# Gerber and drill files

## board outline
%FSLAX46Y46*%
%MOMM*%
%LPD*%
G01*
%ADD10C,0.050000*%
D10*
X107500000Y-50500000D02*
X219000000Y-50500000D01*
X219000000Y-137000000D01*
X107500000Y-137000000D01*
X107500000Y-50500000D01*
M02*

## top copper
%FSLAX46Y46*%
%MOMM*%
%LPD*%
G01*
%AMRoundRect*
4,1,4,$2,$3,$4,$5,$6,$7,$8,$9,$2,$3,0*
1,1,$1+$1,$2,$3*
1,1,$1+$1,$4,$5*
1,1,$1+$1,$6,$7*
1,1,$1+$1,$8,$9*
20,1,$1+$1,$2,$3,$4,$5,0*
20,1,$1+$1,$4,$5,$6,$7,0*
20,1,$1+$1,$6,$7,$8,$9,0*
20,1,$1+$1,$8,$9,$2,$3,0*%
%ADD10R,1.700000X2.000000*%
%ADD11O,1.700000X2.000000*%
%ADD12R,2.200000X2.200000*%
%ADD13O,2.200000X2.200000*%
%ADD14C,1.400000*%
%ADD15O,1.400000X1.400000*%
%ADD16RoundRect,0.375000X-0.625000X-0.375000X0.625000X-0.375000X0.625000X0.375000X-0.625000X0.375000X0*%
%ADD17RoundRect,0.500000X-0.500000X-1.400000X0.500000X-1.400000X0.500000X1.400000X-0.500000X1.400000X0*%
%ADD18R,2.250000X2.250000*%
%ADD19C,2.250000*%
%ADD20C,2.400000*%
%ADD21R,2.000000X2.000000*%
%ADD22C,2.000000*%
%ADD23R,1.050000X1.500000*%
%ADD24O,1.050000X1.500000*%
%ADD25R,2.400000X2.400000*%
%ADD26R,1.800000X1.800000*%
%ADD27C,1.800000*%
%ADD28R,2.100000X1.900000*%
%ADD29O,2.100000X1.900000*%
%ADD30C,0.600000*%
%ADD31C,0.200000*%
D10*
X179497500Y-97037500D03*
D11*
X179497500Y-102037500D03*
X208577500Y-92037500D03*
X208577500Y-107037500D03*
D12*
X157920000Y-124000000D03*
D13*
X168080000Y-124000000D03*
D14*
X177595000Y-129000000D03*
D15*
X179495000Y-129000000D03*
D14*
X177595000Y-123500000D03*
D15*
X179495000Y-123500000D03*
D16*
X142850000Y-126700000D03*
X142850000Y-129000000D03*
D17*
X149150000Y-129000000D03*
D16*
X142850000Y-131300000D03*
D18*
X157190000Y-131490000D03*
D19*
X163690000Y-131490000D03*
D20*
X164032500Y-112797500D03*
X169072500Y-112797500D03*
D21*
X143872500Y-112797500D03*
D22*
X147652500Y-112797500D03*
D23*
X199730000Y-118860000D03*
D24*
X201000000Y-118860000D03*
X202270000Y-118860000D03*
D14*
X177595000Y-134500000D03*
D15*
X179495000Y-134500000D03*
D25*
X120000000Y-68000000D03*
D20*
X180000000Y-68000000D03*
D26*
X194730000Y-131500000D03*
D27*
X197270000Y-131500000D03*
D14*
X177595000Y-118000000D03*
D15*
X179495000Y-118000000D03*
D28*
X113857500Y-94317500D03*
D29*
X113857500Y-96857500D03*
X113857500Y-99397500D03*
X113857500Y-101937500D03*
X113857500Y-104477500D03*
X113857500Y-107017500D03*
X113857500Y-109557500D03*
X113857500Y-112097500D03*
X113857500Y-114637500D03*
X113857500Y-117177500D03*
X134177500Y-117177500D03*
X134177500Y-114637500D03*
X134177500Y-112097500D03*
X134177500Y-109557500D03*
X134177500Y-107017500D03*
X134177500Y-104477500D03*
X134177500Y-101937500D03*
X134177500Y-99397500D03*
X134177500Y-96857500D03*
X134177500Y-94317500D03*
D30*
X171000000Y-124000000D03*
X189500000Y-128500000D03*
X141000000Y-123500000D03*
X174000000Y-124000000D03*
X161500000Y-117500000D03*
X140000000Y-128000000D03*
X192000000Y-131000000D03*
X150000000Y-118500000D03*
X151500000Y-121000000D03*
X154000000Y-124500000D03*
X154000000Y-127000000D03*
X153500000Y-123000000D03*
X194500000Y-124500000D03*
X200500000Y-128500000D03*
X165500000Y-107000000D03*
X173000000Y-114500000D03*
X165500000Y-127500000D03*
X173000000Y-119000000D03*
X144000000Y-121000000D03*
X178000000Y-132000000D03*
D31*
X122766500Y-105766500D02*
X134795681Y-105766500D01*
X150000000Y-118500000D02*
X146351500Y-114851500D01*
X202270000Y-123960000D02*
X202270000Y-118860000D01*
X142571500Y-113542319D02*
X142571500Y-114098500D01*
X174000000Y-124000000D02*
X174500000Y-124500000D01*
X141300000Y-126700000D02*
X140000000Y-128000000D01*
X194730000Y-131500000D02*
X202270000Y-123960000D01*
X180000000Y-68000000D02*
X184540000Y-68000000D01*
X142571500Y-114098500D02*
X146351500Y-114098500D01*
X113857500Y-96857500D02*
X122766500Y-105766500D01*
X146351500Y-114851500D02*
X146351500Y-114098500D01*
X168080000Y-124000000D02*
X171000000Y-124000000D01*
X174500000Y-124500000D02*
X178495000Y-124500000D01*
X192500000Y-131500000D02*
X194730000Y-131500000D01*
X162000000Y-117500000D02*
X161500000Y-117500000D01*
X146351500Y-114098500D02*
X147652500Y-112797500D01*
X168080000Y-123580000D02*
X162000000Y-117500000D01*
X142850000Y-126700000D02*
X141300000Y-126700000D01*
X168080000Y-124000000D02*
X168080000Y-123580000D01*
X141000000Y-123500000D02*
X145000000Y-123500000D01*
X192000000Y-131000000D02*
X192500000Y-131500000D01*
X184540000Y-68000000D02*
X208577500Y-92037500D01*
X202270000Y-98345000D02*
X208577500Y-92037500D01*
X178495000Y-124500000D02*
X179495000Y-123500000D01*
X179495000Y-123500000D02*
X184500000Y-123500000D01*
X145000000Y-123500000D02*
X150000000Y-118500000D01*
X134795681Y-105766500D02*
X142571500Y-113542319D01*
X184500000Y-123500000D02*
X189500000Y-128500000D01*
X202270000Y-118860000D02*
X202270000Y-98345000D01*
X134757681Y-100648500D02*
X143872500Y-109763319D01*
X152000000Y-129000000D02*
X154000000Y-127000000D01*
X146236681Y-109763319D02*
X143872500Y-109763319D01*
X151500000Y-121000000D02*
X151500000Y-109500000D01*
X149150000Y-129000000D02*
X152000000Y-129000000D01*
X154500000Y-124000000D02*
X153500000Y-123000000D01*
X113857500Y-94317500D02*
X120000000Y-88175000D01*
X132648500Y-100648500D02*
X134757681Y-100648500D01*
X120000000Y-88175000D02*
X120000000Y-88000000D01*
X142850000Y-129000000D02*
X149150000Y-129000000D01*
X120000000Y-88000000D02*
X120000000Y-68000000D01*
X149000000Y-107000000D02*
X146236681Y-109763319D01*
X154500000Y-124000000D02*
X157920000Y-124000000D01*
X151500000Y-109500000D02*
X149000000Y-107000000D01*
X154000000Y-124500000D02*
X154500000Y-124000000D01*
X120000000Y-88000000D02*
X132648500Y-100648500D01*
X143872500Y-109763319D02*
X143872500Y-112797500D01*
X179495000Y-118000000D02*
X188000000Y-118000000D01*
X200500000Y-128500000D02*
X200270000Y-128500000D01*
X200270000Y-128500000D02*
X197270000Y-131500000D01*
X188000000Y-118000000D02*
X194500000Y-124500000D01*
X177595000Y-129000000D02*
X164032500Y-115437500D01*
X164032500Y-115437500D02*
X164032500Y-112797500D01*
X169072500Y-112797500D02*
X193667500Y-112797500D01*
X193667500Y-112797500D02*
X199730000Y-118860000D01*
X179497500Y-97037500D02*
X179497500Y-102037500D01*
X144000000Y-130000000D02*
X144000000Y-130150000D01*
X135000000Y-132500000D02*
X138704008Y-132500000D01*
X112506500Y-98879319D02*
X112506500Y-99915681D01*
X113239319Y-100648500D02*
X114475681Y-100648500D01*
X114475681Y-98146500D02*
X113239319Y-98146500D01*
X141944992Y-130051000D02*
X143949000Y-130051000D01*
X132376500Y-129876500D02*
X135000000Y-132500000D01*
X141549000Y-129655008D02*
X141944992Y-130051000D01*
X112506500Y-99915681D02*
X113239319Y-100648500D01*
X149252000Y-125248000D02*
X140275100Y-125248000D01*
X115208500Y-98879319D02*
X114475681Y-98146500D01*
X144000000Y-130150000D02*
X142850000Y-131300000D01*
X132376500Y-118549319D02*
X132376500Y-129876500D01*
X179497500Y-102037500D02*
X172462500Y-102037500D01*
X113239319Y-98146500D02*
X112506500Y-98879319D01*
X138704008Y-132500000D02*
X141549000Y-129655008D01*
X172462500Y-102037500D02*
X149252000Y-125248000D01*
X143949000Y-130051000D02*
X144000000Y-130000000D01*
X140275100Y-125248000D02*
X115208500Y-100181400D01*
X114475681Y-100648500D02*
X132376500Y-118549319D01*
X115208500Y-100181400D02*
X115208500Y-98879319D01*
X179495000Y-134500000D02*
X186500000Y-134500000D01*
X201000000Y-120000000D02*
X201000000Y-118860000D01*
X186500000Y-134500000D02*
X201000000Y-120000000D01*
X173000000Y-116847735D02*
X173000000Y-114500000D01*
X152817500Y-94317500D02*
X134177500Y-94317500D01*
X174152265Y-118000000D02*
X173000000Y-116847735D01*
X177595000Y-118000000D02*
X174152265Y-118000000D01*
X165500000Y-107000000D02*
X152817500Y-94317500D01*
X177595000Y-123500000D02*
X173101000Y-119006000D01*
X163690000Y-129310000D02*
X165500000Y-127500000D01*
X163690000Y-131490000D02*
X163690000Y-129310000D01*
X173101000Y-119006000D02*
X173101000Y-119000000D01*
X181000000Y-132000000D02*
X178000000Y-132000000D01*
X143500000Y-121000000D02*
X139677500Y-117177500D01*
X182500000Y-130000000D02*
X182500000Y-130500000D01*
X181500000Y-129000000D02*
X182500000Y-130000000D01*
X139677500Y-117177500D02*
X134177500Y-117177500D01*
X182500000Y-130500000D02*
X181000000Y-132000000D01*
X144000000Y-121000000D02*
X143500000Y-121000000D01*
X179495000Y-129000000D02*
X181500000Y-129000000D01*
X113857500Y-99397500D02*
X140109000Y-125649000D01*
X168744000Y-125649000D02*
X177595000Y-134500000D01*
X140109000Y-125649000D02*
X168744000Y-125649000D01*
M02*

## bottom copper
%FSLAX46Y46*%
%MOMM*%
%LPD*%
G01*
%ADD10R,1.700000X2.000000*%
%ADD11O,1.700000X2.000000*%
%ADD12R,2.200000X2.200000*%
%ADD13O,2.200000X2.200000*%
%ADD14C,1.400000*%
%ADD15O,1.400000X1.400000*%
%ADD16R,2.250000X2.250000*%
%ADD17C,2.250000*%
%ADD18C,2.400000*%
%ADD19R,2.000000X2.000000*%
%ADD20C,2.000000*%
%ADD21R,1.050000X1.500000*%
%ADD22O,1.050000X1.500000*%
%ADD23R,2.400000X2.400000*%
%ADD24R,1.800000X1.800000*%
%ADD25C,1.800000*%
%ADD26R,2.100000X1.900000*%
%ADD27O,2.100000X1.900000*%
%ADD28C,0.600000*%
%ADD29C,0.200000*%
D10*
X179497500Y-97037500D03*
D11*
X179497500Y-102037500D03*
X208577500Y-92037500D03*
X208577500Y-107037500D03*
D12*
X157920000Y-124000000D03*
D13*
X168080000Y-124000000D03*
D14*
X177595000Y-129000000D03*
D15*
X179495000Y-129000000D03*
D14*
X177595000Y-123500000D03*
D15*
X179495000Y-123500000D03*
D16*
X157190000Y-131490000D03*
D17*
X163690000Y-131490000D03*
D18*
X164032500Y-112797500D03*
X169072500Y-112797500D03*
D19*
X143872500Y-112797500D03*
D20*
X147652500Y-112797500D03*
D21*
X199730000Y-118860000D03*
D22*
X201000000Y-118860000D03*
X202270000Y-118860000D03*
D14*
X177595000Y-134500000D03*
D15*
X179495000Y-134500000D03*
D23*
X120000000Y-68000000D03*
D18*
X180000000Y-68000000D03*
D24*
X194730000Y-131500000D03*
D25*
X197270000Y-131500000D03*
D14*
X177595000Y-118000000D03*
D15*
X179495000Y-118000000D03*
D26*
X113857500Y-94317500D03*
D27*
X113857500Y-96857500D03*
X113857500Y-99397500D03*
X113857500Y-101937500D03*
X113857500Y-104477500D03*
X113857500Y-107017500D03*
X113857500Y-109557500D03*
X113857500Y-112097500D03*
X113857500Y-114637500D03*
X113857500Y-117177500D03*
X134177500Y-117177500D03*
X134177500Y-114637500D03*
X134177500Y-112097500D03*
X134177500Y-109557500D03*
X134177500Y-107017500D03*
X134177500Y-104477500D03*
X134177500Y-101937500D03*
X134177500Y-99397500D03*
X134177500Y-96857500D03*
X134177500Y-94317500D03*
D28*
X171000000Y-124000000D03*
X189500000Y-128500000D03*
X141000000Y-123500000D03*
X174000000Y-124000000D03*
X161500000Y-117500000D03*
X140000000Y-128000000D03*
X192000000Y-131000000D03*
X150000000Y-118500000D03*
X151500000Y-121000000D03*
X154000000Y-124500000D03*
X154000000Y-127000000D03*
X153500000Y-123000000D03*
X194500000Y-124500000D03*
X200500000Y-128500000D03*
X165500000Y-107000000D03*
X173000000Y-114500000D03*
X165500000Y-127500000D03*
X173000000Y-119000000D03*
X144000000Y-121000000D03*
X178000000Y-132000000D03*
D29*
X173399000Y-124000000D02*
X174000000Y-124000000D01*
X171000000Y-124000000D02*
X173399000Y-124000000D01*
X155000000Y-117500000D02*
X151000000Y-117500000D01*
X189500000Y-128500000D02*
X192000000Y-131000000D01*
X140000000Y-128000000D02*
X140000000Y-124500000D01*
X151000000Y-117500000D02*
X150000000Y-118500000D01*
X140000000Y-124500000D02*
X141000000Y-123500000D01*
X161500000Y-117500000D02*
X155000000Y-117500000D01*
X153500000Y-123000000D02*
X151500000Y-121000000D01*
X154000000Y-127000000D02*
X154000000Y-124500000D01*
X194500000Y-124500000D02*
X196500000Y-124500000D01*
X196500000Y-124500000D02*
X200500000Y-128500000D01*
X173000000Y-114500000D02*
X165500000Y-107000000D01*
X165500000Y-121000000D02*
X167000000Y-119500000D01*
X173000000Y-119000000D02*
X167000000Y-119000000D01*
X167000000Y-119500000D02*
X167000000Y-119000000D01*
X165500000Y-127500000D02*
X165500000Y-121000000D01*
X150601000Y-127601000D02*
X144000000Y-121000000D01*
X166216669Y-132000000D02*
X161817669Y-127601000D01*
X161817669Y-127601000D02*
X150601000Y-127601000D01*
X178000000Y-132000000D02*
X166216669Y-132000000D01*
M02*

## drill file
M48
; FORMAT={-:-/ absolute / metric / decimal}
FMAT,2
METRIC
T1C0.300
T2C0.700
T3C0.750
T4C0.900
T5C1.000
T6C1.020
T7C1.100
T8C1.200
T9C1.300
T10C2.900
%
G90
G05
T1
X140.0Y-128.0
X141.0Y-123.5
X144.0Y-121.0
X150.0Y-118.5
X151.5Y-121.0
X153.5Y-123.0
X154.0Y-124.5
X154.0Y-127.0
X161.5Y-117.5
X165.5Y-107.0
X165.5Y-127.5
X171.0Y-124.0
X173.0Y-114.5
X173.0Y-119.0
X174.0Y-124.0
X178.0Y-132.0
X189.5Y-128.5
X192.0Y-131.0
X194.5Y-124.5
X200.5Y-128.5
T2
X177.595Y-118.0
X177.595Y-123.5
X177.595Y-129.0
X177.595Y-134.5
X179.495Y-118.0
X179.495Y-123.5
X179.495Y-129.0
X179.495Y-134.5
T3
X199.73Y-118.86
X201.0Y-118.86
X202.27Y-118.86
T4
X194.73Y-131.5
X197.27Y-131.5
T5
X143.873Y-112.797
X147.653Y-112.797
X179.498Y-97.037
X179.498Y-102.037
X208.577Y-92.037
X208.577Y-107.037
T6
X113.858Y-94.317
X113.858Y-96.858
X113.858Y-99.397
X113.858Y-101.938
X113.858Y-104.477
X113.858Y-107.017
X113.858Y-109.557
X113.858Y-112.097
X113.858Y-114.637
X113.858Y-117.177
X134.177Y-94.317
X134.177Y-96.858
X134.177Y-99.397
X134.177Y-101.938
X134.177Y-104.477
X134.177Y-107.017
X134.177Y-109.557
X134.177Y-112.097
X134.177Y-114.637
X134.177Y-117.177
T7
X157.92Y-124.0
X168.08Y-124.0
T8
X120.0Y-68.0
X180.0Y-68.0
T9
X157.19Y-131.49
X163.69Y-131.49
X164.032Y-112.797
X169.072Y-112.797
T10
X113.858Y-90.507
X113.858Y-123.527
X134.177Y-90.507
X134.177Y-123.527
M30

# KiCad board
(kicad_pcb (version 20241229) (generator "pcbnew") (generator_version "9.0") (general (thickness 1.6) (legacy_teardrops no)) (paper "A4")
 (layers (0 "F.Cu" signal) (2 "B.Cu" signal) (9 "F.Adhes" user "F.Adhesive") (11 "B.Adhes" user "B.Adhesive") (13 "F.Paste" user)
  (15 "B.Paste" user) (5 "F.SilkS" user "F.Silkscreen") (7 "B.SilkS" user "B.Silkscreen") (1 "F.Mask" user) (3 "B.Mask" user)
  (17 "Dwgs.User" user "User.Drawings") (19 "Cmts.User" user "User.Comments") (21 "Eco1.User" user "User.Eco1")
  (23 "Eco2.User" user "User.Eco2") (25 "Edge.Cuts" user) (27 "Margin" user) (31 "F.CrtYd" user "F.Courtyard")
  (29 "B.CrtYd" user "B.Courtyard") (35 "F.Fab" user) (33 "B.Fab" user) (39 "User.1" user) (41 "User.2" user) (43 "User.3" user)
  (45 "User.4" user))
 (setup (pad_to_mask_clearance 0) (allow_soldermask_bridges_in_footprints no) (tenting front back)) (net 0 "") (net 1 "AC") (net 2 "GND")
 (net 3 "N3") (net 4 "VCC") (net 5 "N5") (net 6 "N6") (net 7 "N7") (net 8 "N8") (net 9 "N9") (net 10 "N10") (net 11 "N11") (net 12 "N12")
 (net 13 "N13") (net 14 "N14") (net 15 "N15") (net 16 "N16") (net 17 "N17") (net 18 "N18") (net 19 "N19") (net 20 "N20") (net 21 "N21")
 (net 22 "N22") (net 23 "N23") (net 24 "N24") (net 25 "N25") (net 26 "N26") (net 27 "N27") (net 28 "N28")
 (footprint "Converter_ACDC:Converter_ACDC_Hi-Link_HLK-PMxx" (layer "F.Cu") (at 179.4975 97.0375)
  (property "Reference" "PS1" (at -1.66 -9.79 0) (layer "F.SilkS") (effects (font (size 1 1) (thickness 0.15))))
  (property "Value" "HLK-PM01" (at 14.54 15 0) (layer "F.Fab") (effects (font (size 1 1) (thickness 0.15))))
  (pad "1" thru_hole rect (at 0 0) (size 1.7 2) (drill 1) (layers "*.Cu" "*.Mask") (remove_unused_layers no) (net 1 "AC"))
  (pad "2" thru_hole oval (at 0 5) (size 1.7 2) (drill 1) (layers "*.Cu" "*.Mask") (remove_unused_layers no) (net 1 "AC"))
  (pad "3" thru_hole oval (at 29.08 -5) (size 1.7 2) (drill 1) (layers "*.Cu" "*.Mask") (remove_unused_layers no) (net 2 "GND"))
  (pad "4" thru_hole oval (at 29.08 10) (size 1.7 2) (drill 1) (layers "*.Cu" "*.Mask") (remove_unused_layers no) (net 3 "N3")))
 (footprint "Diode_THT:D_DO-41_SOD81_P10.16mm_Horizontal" (layer "F.Cu") (at 157.92 124)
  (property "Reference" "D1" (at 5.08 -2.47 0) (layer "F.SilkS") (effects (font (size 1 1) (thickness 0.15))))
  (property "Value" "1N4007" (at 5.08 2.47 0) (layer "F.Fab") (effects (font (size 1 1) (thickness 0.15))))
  (pad "1" thru_hole rect (at 0 0) (size 2.2 2.2) (drill 1.1) (layers "*.Cu" "*.Mask") (remove_unused_layers no) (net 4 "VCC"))
  (pad "2" thru_hole oval (at 10.16 0) (size 2.2 2.2) (drill 1.1) (layers "*.Cu" "*.Mask") (remove_unused_layers no) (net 2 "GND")))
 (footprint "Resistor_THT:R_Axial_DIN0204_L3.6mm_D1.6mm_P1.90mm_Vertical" (layer "F.Cu") (at 177.595 129)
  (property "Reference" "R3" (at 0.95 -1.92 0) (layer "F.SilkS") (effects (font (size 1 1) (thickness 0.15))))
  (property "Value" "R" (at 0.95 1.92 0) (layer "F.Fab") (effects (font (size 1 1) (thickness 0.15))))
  (pad "1" thru_hole circle (at 0 0) (size 1.4 1.4) (drill 0.7) (layers "*.Cu" "*.Mask") (remove_unused_layers no) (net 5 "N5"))
  (pad "2" thru_hole oval (at 1.9 0) (size 1.4 1.4) (drill 0.7) (layers "*.Cu" "*.Mask") (remove_unused_layers no) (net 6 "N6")))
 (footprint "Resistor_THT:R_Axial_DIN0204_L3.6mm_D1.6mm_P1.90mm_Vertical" (layer "F.Cu") (at 177.595 123.5)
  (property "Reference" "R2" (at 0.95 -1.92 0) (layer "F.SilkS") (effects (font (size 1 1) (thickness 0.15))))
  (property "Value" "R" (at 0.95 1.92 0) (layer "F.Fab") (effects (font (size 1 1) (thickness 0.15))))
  (pad "1" thru_hole circle (at 0 0) (size 1.4 1.4) (drill 0.7) (layers "*.Cu" "*.Mask") (remove_unused_layers no) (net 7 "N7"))
  (pad "2" thru_hole oval (at 1.9 0) (size 1.4 1.4) (drill 0.7) (layers "*.Cu" "*.Mask") (remove_unused_layers no) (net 2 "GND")))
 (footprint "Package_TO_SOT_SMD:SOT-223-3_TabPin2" (layer "F.Cu") (at 146 129)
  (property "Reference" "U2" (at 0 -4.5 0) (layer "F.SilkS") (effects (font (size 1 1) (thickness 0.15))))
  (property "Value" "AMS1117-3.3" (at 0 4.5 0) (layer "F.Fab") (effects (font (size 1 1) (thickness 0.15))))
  (pad "1" smd roundrect (at -3.15 -2.3) (size 2 1.5) (layers "F.Cu" "F.Mask" "F.Paste") (roundrect_rratio 0.25) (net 2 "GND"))
  (pad "2" smd roundrect (at -3.15 0) (size 2 1.5) (layers "F.Cu" "F.Mask" "F.Paste") (roundrect_rratio 0.25) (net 4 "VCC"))
  (pad "2" smd roundrect (at 3.15 0) (size 2 3.8) (layers "F.Cu" "F.Mask" "F.Paste") (roundrect_rratio 0.25) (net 4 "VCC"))
  (pad "3" smd roundrect (at -3.15 2.3) (size 2 1.5) (layers "F.Cu" "F.Mask" "F.Paste") (roundrect_rratio 0.25) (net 1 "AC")))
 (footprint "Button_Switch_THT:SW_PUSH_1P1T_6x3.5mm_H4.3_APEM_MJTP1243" (layer "F.Cu") (at 157.19 131.49)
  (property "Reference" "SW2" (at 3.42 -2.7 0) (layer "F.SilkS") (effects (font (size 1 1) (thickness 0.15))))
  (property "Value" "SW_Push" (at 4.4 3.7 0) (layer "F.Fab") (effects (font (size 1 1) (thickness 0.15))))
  (pad "1" thru_hole rect (at 0 0 90) (size 2.25 2.25) (drill 1.3) (layers "*.Cu" "*.Mask") (remove_unused_layers no) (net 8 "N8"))
  (pad "2" thru_hole circle (at 6.5 0 90) (size 2.25 2.25) (drill 1.3) (layers "*.Cu" "*.Mask") (remove_unused_layers no) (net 7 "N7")))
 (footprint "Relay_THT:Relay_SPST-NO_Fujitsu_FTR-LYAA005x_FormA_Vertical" (layer "F.Cu") (at 143.8725 112.7975)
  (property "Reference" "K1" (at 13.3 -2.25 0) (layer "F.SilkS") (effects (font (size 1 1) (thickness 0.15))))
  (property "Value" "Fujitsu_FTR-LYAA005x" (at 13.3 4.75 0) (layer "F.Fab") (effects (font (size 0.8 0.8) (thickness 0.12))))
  (pad "13" thru_hole circle (at 20.16 0) (size 2.4 2.4) (drill 1.3) (layers "*.Cu" "*.Mask") (remove_unused_layers no) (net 5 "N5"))
  (pad "14" thru_hole circle (at 25.2 0) (size 2.4 2.4) (drill 1.3) (layers "*.Cu" "*.Mask") (remove_unused_layers no) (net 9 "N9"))
  (pad "A1" thru_hole rect (at 0 0) (size 2 2) (drill 1) (layers "*.Cu" "*.Mask") (remove_unused_layers no) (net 4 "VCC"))
  (pad "A2" thru_hole circle (at 3.78 0) (size 2 2) (drill 1) (layers "*.Cu" "*.Mask") (remove_unused_layers no) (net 2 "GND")))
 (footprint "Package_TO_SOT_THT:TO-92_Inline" (layer "F.Cu") (at 199.73 118.86)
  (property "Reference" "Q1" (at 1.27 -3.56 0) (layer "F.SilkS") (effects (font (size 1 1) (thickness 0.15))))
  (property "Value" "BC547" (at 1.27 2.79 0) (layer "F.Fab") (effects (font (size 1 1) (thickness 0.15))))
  (pad "1" thru_hole rect (at 0 0) (size 1.05 1.5) (drill 0.75) (layers "*.Cu" "*.Mask") (remove_unused_layers no) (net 9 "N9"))
  (pad "2" thru_hole oval (at 1.27 0) (size 1.05 1.5) (drill 0.75) (layers "*.Cu" "*.Mask") (remove_unused_layers no) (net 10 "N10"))
  (pad "3" thru_hole oval (at 2.54 0) (size 1.05 1.5) (drill 0.75) (layers "*.Cu" "*.Mask") (remove_unused_layers no) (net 2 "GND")))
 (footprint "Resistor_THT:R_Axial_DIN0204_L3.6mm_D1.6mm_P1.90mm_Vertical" (layer "F.Cu") (at 177.595 134.5)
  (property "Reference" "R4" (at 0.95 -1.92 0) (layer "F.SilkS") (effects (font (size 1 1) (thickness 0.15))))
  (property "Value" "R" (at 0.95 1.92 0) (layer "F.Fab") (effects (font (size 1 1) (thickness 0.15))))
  (pad "1" thru_hole circle (at 0 0) (size 1.4 1.4) (drill 0.7) (layers "*.Cu" "*.Mask") (remove_unused_layers no) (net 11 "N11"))
  (pad "2" thru_hole oval (at 1.9 0) (size 1.4 1.4) (drill 0.7) (layers "*.Cu" "*.Mask") (remove_unused_layers no) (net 10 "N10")))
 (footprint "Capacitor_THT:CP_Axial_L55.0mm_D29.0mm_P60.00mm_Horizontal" (layer "F.Cu") (at 120 68)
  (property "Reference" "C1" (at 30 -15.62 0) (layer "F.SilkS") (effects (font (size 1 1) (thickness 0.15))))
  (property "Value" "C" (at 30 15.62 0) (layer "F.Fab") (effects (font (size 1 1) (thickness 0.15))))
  (pad "1" thru_hole rect (at 0 0) (size 2.4 2.4) (drill 1.2) (layers "*.Cu" "*.Mask") (remove_unused_layers no) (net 4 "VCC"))
  (pad "2" thru_hole circle (at 60 0) (size 2.4 2.4) (drill 1.2) (layers "*.Cu" "*.Mask") (remove_unused_layers no) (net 2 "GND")))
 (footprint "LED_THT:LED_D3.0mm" (layer "F.Cu") (at 194.73 131.5)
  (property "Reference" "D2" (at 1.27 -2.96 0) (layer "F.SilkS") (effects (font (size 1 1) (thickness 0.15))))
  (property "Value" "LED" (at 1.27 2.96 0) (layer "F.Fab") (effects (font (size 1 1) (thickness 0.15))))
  (pad "1" thru_hole rect (at 0 0) (size 1.8 1.8) (drill 0.9) (layers "*.Cu" "*.Mask") (remove_unused_layers no) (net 2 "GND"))
  (pad "2" thru_hole circle (at 2.54 0) (size 1.8 1.8) (drill 0.9) (layers "*.Cu" "*.Mask") (remove_unused_layers no) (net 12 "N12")))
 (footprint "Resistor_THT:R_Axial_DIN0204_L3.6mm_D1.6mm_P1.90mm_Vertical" (layer "F.Cu") (at 177.595 118)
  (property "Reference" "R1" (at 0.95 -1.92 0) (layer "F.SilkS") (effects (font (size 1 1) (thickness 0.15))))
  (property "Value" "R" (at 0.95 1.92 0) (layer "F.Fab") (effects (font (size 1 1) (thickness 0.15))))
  (pad "1" thru_hole circle (at 0 0) (size 1.4 1.4) (drill 0.7) (layers "*.Cu" "*.Mask") (remove_unused_layers no) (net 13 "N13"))
  (pad "2" thru_hole oval (at 1.9 0) (size 1.4 1.4) (drill 0.7) (layers "*.Cu" "*.Mask") (remove_unused_layers no) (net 12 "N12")))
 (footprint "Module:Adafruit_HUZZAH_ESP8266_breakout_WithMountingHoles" (layer "F.Cu") (at 113.8575 94.3175)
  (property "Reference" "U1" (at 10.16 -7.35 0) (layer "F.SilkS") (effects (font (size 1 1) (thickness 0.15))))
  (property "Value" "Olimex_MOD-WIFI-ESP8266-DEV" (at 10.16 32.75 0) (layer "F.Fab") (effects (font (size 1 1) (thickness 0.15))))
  (pad "" np_thru_hole circle (at 0 -3.81) (size 2.9 2.9) (drill 2.9) (layers "*.Cu" "*.Mask"))
  (pad "" np_thru_hole circle (at 0 29.21) (size 2.9 2.9) (drill 2.9) (layers "*.Cu" "*.Mask"))
  (pad "" np_thru_hole circle (at 20.32 -3.81) (size 2.9 2.9) (drill 2.9) (layers "*.Cu" "*.Mask"))
  (pad "" np_thru_hole circle (at 20.32 29.21) (size 2.9 2.9) (drill 2.9) (layers "*.Cu" "*.Mask"))
  (pad "1" thru_hole rect (at 0 0) (size 2.1 1.9) (drill 1.02) (layers "*.Cu" "*.Mask") (remove_unused_layers no) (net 4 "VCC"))
  (pad "2" thru_hole oval (at 0 2.54) (size 2.1 1.9) (drill 1.02) (layers "*.Cu" "*.Mask") (remove_unused_layers no) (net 2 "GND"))
  (pad "3" thru_hole oval (at 0 5.08) (size 2.1 1.9) (drill 1.02) (layers "*.Cu" "*.Mask") (remove_unused_layers no) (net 11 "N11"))
  (pad "4" thru_hole oval (at 0 7.62) (size 2.1 1.9) (drill 1.02) (layers "*.Cu" "*.Mask") (remove_unused_layers no) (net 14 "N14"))
  (pad "5" thru_hole oval (at 0 10.16) (size 2.1 1.9) (drill 1.02) (layers "*.Cu" "*.Mask") (remove_unused_layers no) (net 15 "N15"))
  (pad "6" thru_hole oval (at 0 12.7) (size 2.1 1.9) (drill 1.02) (layers "*.Cu" "*.Mask") (remove_unused_layers no) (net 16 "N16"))
  (pad "7" thru_hole oval (at 0 15.24) (size 2.1 1.9) (drill 1.02) (layers "*.Cu" "*.Mask") (remove_unused_layers no) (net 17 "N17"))
  (pad "8" thru_hole oval (at 0 17.78) (size 2.1 1.9) (drill 1.02) (layers "*.Cu" "*.Mask") (remove_unused_layers no) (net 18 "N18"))
  (pad "9" thru_hole oval (at 0 20.32) (size 2.1 1.9) (drill 1.02) (layers "*.Cu" "*.Mask") (remove_unused_layers no) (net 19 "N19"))
  (pad "10" thru_hole oval (at 0 22.86) (size 2.1 1.9) (drill 1.02) (layers "*.Cu" "*.Mask") (remove_unused_layers no) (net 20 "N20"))
  (pad "11" thru_hole oval (at 20.32 22.86) (size 2.1 1.9) (drill 1.02) (layers "*.Cu" "*.Mask") (remove_unused_layers no) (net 6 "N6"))
  (pad "12" thru_hole oval (at 20.32 20.32) (size 2.1 1.9) (drill 1.02) (layers "*.Cu" "*.Mask") (remove_unused_layers no) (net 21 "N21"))
  (pad "13" thru_hole oval (at 20.32 17.78) (size 2.1 1.9) (drill 1.02) (layers "*.Cu" "*.Mask") (remove_unused_layers no) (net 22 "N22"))
  (pad "14" thru_hole oval (at 20.32 15.24) (size 2.1 1.9) (drill 1.02) (layers "*.Cu" "*.Mask") (remove_unused_layers no) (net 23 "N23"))
  (pad "15" thru_hole oval (at 20.32 12.7) (size 2.1 1.9) (drill 1.02) (layers "*.Cu" "*.Mask") (remove_unused_layers no) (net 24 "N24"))
  (pad "16" thru_hole oval (at 20.32 10.16) (size 2.1 1.9) (drill 1.02) (layers "*.Cu" "*.Mask") (remove_unused_layers no) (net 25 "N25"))
  (pad "17" thru_hole oval (at 20.32 7.62) (size 2.1 1.9) (drill 1.02) (layers "*.Cu" "*.Mask") (remove_unused_layers no) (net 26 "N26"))
  (pad "18" thru_hole oval (at 20.32 5.08) (size 2.1 1.9) (drill 1.02) (layers "*.Cu" "*.Mask") (remove_unused_layers no) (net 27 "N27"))
  (pad "19" thru_hole oval (at 20.32 2.54) (size 2.1 1.9) (drill 1.02) (layers "*.Cu" "*.Mask") (remove_unused_layers no) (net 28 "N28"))
  (pad "20" thru_hole oval (at 20.32 0) (size 2.1 1.9) (drill 1.02) (layers "*.Cu" "*.Mask") (remove_unused_layers no) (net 13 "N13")))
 (gr_rect (start 107.5 50.5) (end 219 137) (stroke (width 0.05) (type default)) (fill no) (layer "Edge.Cuts"))
 (segment (start 122.7665 105.7665) (end 134.795681 105.7665) (width 0.2) (layer "F.Cu") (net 2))
 (segment (start 150 118.5) (end 146.3515 114.8515) (width 0.2) (layer "F.Cu") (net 2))
 (segment (start 202.27 123.96) (end 202.27 118.86) (width 0.2) (layer "F.Cu") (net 2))
 (segment (start 142.5715 113.542319) (end 142.5715 114.0985) (width 0.2) (layer "F.Cu") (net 2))
 (segment (start 174 124) (end 174.5 124.5) (width 0.2) (layer "F.Cu") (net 2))
 (segment (start 141.3 126.7) (end 140 128) (width 0.2) (layer "F.Cu") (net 2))
 (segment (start 194.73 131.5) (end 202.27 123.96) (width 0.2) (layer "F.Cu") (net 2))
 (segment (start 180 68) (end 184.54 68) (width 0.2) (layer "F.Cu") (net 2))
 (segment (start 142.5715 114.0985) (end 146.3515 114.0985) (width 0.2) (layer "F.Cu") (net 2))
 (segment (start 113.8575 96.8575) (end 122.7665 105.7665) (width 0.2) (layer "F.Cu") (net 2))
 (segment (start 146.3515 114.8515) (end 146.3515 114.0985) (width 0.2) (layer "F.Cu") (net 2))
 (segment (start 168.08 124) (end 171 124) (width 0.2) (layer "F.Cu") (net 2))
 (segment (start 174.5 124.5) (end 178.495 124.5) (width 0.2) (layer "F.Cu") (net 2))
 (segment (start 192.5 131.5) (end 194.73 131.5) (width 0.2) (layer "F.Cu") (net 2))
 (segment (start 162 117.5) (end 161.5 117.5) (width 0.2) (layer "F.Cu") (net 2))
 (segment (start 146.3515 114.0985) (end 147.6525 112.7975) (width 0.2) (layer "F.Cu") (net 2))
 (segment (start 168.08 123.58) (end 162 117.5) (width 0.2) (layer "F.Cu") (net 2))
 (segment (start 142.85 126.7) (end 141.3 126.7) (width 0.2) (layer "F.Cu") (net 2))
 (segment (start 168.08 124) (end 168.08 123.58) (width 0.2) (layer "F.Cu") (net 2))
 (segment (start 141 123.5) (end 145 123.5) (width 0.2) (layer "F.Cu") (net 2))
 (segment (start 192 131) (end 192.5 131.5) (width 0.2) (layer "F.Cu") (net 2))
 (segment (start 184.54 68) (end 208.5775 92.0375) (width 0.2) (layer "F.Cu") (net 2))
 (segment (start 202.27 98.345) (end 208.5775 92.0375) (width 0.2) (layer "F.Cu") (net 2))
 (segment (start 178.495 124.5) (end 179.495 123.5) (width 0.2) (layer "F.Cu") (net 2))
 (segment (start 179.495 123.5) (end 184.5 123.5) (width 0.2) (layer "F.Cu") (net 2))
 (segment (start 145 123.5) (end 150 118.5) (width 0.2) (layer "F.Cu") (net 2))
 (segment (start 134.795681 105.7665) (end 142.5715 113.542319) (width 0.2) (layer "F.Cu") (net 2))
 (segment (start 184.5 123.5) (end 189.5 128.5) (width 0.2) (layer "F.Cu") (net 2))
 (segment (start 202.27 118.86) (end 202.27 98.345) (width 0.2) (layer "F.Cu") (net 2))
 (via (at 171 124) (size 0.6) (drill 0.3) (layers "F.Cu" "B.Cu") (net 2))
 (via (at 189.5 128.5) (size 0.6) (drill 0.3) (layers "F.Cu" "B.Cu") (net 2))
 (via (at 141 123.5) (size 0.6) (drill 0.3) (layers "F.Cu" "B.Cu") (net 2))
 (via (at 174 124) (size 0.6) (drill 0.3) (layers "F.Cu" "B.Cu") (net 2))
 (via (at 161.5 117.5) (size 0.6) (drill 0.3) (layers "F.Cu" "B.Cu") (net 2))
 (via (at 140 128) (size 0.6) (drill 0.3) (layers "F.Cu" "B.Cu") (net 2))
 (via (at 192 131) (size 0.6) (drill 0.3) (layers "F.Cu" "B.Cu") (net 2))
 (via (at 150 118.5) (size 0.6) (drill 0.3) (layers "F.Cu" "B.Cu") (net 2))
 (segment (start 173.399 124) (end 174 124) (width 0.2) (layer "B.Cu") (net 2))
 (segment (start 171 124) (end 173.399 124) (width 0.2) (layer "B.Cu") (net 2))
 (segment (start 155 117.5) (end 151 117.5) (width 0.2) (layer "B.Cu") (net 2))
 (segment (start 189.5 128.5) (end 192 131) (width 0.2) (layer "B.Cu") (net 2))
 (segment (start 140 128) (end 140 124.5) (width 0.2) (layer "B.Cu") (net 2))
 (segment (start 151 117.5) (end 150 118.5) (width 0.2) (layer "B.Cu") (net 2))
 (segment (start 140 124.5) (end 141 123.5) (width 0.2) (layer "B.Cu") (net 2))
 (segment (start 161.5 117.5) (end 155 117.5) (width 0.2) (layer "B.Cu") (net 2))
 (segment (start 134.757681 100.6485) (end 143.8725 109.763319) (width 0.2) (layer "F.Cu") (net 4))
 (segment (start 152 129) (end 154 127) (width 0.2) (layer "F.Cu") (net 4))
 (segment (start 146.236681 109.763319) (end 143.8725 109.763319) (width 0.2) (layer "F.Cu") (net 4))
 (segment (start 151.5 121) (end 151.5 109.5) (width 0.2) (layer "F.Cu") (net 4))
 (segment (start 149.15 129) (end 152 129) (width 0.2) (layer "F.Cu") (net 4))
 (segment (start 154.5 124) (end 153.5 123) (width 0.2) (layer "F.Cu") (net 4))
 (segment (start 113.8575 94.3175) (end 120 88.175) (width 0.2) (layer "F.Cu") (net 4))
 (segment (start 132.6485 100.6485) (end 134.757681 100.6485) (width 0.2) (layer "F.Cu") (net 4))
 (segment (start 120 88.175) (end 120 88) (width 0.2) (layer "F.Cu") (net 4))
 (segment (start 142.85 129) (end 149.15 129) (width 0.2) (layer "F.Cu") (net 4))
 (segment (start 120 88) (end 120 68) (width 0.2) (layer "F.Cu") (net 4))
 (segment (start 149 107) (end 146.236681 109.763319) (width 0.2) (layer "F.Cu") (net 4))
 (segment (start 154.5 124) (end 157.92 124) (width 0.2) (layer "F.Cu") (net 4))
 (segment (start 151.5 109.5) (end 149 107) (width 0.2) (layer "F.Cu") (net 4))
 (segment (start 154 124.5) (end 154.5 124) (width 0.2) (layer "F.Cu") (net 4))
 (segment (start 120 88) (end 132.6485 100.6485) (width 0.2) (layer "F.Cu") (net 4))
 (segment (start 143.8725 109.763319) (end 143.8725 112.7975) (width 0.2) (layer "F.Cu") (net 4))
 (via (at 151.5 121) (size 0.6) (drill 0.3) (layers "F.Cu" "B.Cu") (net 4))
 (via (at 154 124.5) (size 0.6) (drill 0.3) (layers "F.Cu" "B.Cu") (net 4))
 (via (at 154 127) (size 0.6) (drill 0.3) (layers "F.Cu" "B.Cu") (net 4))
 (via (at 153.5 123) (size 0.6) (drill 0.3) (layers "F.Cu" "B.Cu") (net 4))
 (segment (start 153.5 123) (end 151.5 121) (width 0.2) (layer "B.Cu") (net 4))
 (segment (start 154 127) (end 154 124.5) (width 0.2) (layer "B.Cu") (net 4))
 (segment (start 179.495 118) (end 188 118) (width 0.2) (layer "F.Cu") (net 12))
 (segment (start 200.5 128.5) (end 200.27 128.5) (width 0.2) (layer "F.Cu") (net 12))
 (segment (start 200.27 128.5) (end 197.27 131.5) (width 0.2) (layer "F.Cu") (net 12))
 (segment (start 188 118) (end 194.5 124.5) (width 0.2) (layer "F.Cu") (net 12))
 (via (at 194.5 124.5) (size 0.6) (drill 0.3) (layers "F.Cu" "B.Cu") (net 12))
 (via (at 200.5 128.5) (size 0.6) (drill 0.3) (layers "F.Cu" "B.Cu") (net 12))
 (segment (start 194.5 124.5) (end 196.5 124.5) (width 0.2) (layer "B.Cu") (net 12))
 (segment (start 196.5 124.5) (end 200.5 128.5) (width 0.2) (layer "B.Cu") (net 12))
 (segment (start 177.595 129) (end 164.0325 115.4375) (width 0.2) (layer "F.Cu") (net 5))
 (segment (start 164.0325 115.4375) (end 164.0325 112.7975) (width 0.2) (layer "F.Cu") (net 5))
 (segment (start 169.0725 112.7975) (end 193.6675 112.7975) (width 0.2) (layer "F.Cu") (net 9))
 (segment (start 193.6675 112.7975) (end 199.73 118.86) (width 0.2) (layer "F.Cu") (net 9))
 (segment (start 179.4975 97.0375) (end 179.4975 102.0375) (width 0.2) (layer "F.Cu") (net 1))
 (segment (start 144 130) (end 144 130.15) (width 0.2) (layer "F.Cu") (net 1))
 (segment (start 135 132.5) (end 138.704008 132.5) (width 0.2) (layer "F.Cu") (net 1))
 (segment (start 112.5065 98.879319) (end 112.5065 99.915681) (width 0.2) (layer "F.Cu") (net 1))
 (segment (start 113.239319 100.6485) (end 114.475681 100.6485) (width 0.2) (layer "F.Cu") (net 1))
 (segment (start 114.475681 98.1465) (end 113.239319 98.1465) (width 0.2) (layer "F.Cu") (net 1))
 (segment (start 141.944992 130.051) (end 143.949 130.051) (width 0.2) (layer "F.Cu") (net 1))
 (segment (start 132.3765 129.8765) (end 135 132.5) (width 0.2) (layer "F.Cu") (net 1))
 (segment (start 141.549 129.655008) (end 141.944992 130.051) (width 0.2) (layer "F.Cu") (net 1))
 (segment (start 112.5065 99.915681) (end 113.239319 100.6485) (width 0.2) (layer "F.Cu") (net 1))
 (segment (start 149.252 125.248) (end 140.2751 125.248) (width 0.2) (layer "F.Cu") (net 1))
 (segment (start 115.2085 98.879319) (end 114.475681 98.1465) (width 0.2) (layer "F.Cu") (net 1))
 (segment (start 144 130.15) (end 142.85 131.3) (width 0.2) (layer "F.Cu") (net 1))
 (segment (start 132.3765 118.549319) (end 132.3765 129.8765) (width 0.2) (layer "F.Cu") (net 1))
 (segment (start 179.4975 102.0375) (end 172.4625 102.0375) (width 0.2) (layer "F.Cu") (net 1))
 (segment (start 113.239319 98.1465) (end 112.5065 98.879319) (width 0.2) (layer "F.Cu") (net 1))
 (segment (start 138.704008 132.5) (end 141.549 129.655008) (width 0.2) (layer "F.Cu") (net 1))
 (segment (start 172.4625 102.0375) (end 149.252 125.248) (width 0.2) (layer "F.Cu") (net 1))
 (segment (start 143.949 130.051) (end 144 130) (width 0.2) (layer "F.Cu") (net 1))
 (segment (start 140.2751 125.248) (end 115.2085 100.1814) (width 0.2) (layer "F.Cu") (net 1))
 (segment (start 114.475681 100.6485) (end 132.3765 118.549319) (width 0.2) (layer "F.Cu") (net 1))
 (segment (start 115.2085 100.1814) (end 115.2085 98.879319) (width 0.2) (layer "F.Cu") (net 1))
 (segment (start 179.495 134.5) (end 186.5 134.5) (width 0.2) (layer "F.Cu") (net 10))
 (segment (start 201 120) (end 201 118.86) (width 0.2) (layer "F.Cu") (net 10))
 (segment (start 186.5 134.5) (end 201 120) (width 0.2) (layer "F.Cu") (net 10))
 (segment (start 173 116.847735) (end 173 114.5) (width 0.2) (layer "F.Cu") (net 13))
 (segment (start 152.8175 94.3175) (end 134.1775 94.3175) (width 0.2) (layer "F.Cu") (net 13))
 (segment (start 174.152265 118) (end 173 116.847735) (width 0.2) (layer "F.Cu") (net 13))
 (segment (start 177.595 118) (end 174.152265 118) (width 0.2) (layer "F.Cu") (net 13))
 (segment (start 165.5 107) (end 152.8175 94.3175) (width 0.2) (layer "F.Cu") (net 13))
 (via (at 165.5 107) (size 0.6) (drill 0.3) (layers "F.Cu" "B.Cu") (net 13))
 (via (at 173 114.5) (size 0.6) (drill 0.3) (layers "F.Cu" "B.Cu") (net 13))
 (segment (start 173 114.5) (end 165.5 107) (width 0.2) (layer "B.Cu") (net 13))
 (segment (start 177.595 123.5) (end 173.101 119.006) (width 0.2) (layer "F.Cu") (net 7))
 (segment (start 163.69 129.31) (end 165.5 127.5) (width 0.2) (layer "F.Cu") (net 7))
 (segment (start 163.69 131.49) (end 163.69 129.31) (width 0.2) (layer "F.Cu") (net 7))
 (segment (start 173.101 119.006) (end 173.101 119) (width 0.2) (layer "F.Cu") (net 7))
 (via (at 165.5 127.5) (size 0.6) (drill 0.3) (layers "F.Cu" "B.Cu") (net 7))
 (via (at 173 119) (size 0.6) (drill 0.3) (layers "F.Cu" "B.Cu") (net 7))
 (segment (start 165.5 121) (end 167 119.5) (width 0.2) (layer "B.Cu") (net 7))
 (segment (start 173 119) (end 167 119) (width 0.2) (layer "B.Cu") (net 7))
 (segment (start 167 119.5) (end 167 119) (width 0.2) (layer "B.Cu") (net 7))
 (segment (start 165.5 127.5) (end 165.5 121) (width 0.2) (layer "B.Cu") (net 7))
 (segment (start 181 132) (end 178 132) (width 0.2) (layer "F.Cu") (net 6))
 (segment (start 143.5 121) (end 139.6775 117.1775) (width 0.2) (layer "F.Cu") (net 6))
 (segment (start 182.5 130) (end 182.5 130.5) (width 0.2) (layer "F.Cu") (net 6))
 (segment (start 181.5 129) (end 182.5 130) (width 0.2) (layer "F.Cu") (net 6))
 (segment (start 139.6775 117.1775) (end 134.1775 117.1775) (width 0.2) (layer "F.Cu") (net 6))
 (segment (start 182.5 130.5) (end 181 132) (width 0.2) (layer "F.Cu") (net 6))
 (segment (start 144 121) (end 143.5 121) (width 0.2) (layer "F.Cu") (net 6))
 (segment (start 179.495 129) (end 181.5 129) (width 0.2) (layer "F.Cu") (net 6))
 (via (at 144 121) (size 0.6) (drill 0.3) (layers "F.Cu" "B.Cu") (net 6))
 (via (at 178 132) (size 0.6) (drill 0.3) (layers "F.Cu" "B.Cu") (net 6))
 (segment (start 150.601 127.601) (end 144 121) (width 0.2) (layer "B.Cu") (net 6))
 (segment (start 166.216669 132) (end 161.817669 127.601) (width 0.2) (layer "B.Cu") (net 6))
 (segment (start 161.817669 127.601) (end 150.601 127.601) (width 0.2) (layer "B.Cu") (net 6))
 (segment (start 178 132) (end 166.216669 132) (width 0.2) (layer "B.Cu") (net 6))
 (segment (start 113.8575 99.3975) (end 140.109 125.649) (width 0.2) (layer "F.Cu") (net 11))
 (segment (start 168.744 125.649) (end 177.595 134.5) (width 0.2) (layer "F.Cu") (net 11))
 (segment (start 140.109 125.649) (end 168.744 125.649) (width 0.2) (layer "F.Cu") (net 11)))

